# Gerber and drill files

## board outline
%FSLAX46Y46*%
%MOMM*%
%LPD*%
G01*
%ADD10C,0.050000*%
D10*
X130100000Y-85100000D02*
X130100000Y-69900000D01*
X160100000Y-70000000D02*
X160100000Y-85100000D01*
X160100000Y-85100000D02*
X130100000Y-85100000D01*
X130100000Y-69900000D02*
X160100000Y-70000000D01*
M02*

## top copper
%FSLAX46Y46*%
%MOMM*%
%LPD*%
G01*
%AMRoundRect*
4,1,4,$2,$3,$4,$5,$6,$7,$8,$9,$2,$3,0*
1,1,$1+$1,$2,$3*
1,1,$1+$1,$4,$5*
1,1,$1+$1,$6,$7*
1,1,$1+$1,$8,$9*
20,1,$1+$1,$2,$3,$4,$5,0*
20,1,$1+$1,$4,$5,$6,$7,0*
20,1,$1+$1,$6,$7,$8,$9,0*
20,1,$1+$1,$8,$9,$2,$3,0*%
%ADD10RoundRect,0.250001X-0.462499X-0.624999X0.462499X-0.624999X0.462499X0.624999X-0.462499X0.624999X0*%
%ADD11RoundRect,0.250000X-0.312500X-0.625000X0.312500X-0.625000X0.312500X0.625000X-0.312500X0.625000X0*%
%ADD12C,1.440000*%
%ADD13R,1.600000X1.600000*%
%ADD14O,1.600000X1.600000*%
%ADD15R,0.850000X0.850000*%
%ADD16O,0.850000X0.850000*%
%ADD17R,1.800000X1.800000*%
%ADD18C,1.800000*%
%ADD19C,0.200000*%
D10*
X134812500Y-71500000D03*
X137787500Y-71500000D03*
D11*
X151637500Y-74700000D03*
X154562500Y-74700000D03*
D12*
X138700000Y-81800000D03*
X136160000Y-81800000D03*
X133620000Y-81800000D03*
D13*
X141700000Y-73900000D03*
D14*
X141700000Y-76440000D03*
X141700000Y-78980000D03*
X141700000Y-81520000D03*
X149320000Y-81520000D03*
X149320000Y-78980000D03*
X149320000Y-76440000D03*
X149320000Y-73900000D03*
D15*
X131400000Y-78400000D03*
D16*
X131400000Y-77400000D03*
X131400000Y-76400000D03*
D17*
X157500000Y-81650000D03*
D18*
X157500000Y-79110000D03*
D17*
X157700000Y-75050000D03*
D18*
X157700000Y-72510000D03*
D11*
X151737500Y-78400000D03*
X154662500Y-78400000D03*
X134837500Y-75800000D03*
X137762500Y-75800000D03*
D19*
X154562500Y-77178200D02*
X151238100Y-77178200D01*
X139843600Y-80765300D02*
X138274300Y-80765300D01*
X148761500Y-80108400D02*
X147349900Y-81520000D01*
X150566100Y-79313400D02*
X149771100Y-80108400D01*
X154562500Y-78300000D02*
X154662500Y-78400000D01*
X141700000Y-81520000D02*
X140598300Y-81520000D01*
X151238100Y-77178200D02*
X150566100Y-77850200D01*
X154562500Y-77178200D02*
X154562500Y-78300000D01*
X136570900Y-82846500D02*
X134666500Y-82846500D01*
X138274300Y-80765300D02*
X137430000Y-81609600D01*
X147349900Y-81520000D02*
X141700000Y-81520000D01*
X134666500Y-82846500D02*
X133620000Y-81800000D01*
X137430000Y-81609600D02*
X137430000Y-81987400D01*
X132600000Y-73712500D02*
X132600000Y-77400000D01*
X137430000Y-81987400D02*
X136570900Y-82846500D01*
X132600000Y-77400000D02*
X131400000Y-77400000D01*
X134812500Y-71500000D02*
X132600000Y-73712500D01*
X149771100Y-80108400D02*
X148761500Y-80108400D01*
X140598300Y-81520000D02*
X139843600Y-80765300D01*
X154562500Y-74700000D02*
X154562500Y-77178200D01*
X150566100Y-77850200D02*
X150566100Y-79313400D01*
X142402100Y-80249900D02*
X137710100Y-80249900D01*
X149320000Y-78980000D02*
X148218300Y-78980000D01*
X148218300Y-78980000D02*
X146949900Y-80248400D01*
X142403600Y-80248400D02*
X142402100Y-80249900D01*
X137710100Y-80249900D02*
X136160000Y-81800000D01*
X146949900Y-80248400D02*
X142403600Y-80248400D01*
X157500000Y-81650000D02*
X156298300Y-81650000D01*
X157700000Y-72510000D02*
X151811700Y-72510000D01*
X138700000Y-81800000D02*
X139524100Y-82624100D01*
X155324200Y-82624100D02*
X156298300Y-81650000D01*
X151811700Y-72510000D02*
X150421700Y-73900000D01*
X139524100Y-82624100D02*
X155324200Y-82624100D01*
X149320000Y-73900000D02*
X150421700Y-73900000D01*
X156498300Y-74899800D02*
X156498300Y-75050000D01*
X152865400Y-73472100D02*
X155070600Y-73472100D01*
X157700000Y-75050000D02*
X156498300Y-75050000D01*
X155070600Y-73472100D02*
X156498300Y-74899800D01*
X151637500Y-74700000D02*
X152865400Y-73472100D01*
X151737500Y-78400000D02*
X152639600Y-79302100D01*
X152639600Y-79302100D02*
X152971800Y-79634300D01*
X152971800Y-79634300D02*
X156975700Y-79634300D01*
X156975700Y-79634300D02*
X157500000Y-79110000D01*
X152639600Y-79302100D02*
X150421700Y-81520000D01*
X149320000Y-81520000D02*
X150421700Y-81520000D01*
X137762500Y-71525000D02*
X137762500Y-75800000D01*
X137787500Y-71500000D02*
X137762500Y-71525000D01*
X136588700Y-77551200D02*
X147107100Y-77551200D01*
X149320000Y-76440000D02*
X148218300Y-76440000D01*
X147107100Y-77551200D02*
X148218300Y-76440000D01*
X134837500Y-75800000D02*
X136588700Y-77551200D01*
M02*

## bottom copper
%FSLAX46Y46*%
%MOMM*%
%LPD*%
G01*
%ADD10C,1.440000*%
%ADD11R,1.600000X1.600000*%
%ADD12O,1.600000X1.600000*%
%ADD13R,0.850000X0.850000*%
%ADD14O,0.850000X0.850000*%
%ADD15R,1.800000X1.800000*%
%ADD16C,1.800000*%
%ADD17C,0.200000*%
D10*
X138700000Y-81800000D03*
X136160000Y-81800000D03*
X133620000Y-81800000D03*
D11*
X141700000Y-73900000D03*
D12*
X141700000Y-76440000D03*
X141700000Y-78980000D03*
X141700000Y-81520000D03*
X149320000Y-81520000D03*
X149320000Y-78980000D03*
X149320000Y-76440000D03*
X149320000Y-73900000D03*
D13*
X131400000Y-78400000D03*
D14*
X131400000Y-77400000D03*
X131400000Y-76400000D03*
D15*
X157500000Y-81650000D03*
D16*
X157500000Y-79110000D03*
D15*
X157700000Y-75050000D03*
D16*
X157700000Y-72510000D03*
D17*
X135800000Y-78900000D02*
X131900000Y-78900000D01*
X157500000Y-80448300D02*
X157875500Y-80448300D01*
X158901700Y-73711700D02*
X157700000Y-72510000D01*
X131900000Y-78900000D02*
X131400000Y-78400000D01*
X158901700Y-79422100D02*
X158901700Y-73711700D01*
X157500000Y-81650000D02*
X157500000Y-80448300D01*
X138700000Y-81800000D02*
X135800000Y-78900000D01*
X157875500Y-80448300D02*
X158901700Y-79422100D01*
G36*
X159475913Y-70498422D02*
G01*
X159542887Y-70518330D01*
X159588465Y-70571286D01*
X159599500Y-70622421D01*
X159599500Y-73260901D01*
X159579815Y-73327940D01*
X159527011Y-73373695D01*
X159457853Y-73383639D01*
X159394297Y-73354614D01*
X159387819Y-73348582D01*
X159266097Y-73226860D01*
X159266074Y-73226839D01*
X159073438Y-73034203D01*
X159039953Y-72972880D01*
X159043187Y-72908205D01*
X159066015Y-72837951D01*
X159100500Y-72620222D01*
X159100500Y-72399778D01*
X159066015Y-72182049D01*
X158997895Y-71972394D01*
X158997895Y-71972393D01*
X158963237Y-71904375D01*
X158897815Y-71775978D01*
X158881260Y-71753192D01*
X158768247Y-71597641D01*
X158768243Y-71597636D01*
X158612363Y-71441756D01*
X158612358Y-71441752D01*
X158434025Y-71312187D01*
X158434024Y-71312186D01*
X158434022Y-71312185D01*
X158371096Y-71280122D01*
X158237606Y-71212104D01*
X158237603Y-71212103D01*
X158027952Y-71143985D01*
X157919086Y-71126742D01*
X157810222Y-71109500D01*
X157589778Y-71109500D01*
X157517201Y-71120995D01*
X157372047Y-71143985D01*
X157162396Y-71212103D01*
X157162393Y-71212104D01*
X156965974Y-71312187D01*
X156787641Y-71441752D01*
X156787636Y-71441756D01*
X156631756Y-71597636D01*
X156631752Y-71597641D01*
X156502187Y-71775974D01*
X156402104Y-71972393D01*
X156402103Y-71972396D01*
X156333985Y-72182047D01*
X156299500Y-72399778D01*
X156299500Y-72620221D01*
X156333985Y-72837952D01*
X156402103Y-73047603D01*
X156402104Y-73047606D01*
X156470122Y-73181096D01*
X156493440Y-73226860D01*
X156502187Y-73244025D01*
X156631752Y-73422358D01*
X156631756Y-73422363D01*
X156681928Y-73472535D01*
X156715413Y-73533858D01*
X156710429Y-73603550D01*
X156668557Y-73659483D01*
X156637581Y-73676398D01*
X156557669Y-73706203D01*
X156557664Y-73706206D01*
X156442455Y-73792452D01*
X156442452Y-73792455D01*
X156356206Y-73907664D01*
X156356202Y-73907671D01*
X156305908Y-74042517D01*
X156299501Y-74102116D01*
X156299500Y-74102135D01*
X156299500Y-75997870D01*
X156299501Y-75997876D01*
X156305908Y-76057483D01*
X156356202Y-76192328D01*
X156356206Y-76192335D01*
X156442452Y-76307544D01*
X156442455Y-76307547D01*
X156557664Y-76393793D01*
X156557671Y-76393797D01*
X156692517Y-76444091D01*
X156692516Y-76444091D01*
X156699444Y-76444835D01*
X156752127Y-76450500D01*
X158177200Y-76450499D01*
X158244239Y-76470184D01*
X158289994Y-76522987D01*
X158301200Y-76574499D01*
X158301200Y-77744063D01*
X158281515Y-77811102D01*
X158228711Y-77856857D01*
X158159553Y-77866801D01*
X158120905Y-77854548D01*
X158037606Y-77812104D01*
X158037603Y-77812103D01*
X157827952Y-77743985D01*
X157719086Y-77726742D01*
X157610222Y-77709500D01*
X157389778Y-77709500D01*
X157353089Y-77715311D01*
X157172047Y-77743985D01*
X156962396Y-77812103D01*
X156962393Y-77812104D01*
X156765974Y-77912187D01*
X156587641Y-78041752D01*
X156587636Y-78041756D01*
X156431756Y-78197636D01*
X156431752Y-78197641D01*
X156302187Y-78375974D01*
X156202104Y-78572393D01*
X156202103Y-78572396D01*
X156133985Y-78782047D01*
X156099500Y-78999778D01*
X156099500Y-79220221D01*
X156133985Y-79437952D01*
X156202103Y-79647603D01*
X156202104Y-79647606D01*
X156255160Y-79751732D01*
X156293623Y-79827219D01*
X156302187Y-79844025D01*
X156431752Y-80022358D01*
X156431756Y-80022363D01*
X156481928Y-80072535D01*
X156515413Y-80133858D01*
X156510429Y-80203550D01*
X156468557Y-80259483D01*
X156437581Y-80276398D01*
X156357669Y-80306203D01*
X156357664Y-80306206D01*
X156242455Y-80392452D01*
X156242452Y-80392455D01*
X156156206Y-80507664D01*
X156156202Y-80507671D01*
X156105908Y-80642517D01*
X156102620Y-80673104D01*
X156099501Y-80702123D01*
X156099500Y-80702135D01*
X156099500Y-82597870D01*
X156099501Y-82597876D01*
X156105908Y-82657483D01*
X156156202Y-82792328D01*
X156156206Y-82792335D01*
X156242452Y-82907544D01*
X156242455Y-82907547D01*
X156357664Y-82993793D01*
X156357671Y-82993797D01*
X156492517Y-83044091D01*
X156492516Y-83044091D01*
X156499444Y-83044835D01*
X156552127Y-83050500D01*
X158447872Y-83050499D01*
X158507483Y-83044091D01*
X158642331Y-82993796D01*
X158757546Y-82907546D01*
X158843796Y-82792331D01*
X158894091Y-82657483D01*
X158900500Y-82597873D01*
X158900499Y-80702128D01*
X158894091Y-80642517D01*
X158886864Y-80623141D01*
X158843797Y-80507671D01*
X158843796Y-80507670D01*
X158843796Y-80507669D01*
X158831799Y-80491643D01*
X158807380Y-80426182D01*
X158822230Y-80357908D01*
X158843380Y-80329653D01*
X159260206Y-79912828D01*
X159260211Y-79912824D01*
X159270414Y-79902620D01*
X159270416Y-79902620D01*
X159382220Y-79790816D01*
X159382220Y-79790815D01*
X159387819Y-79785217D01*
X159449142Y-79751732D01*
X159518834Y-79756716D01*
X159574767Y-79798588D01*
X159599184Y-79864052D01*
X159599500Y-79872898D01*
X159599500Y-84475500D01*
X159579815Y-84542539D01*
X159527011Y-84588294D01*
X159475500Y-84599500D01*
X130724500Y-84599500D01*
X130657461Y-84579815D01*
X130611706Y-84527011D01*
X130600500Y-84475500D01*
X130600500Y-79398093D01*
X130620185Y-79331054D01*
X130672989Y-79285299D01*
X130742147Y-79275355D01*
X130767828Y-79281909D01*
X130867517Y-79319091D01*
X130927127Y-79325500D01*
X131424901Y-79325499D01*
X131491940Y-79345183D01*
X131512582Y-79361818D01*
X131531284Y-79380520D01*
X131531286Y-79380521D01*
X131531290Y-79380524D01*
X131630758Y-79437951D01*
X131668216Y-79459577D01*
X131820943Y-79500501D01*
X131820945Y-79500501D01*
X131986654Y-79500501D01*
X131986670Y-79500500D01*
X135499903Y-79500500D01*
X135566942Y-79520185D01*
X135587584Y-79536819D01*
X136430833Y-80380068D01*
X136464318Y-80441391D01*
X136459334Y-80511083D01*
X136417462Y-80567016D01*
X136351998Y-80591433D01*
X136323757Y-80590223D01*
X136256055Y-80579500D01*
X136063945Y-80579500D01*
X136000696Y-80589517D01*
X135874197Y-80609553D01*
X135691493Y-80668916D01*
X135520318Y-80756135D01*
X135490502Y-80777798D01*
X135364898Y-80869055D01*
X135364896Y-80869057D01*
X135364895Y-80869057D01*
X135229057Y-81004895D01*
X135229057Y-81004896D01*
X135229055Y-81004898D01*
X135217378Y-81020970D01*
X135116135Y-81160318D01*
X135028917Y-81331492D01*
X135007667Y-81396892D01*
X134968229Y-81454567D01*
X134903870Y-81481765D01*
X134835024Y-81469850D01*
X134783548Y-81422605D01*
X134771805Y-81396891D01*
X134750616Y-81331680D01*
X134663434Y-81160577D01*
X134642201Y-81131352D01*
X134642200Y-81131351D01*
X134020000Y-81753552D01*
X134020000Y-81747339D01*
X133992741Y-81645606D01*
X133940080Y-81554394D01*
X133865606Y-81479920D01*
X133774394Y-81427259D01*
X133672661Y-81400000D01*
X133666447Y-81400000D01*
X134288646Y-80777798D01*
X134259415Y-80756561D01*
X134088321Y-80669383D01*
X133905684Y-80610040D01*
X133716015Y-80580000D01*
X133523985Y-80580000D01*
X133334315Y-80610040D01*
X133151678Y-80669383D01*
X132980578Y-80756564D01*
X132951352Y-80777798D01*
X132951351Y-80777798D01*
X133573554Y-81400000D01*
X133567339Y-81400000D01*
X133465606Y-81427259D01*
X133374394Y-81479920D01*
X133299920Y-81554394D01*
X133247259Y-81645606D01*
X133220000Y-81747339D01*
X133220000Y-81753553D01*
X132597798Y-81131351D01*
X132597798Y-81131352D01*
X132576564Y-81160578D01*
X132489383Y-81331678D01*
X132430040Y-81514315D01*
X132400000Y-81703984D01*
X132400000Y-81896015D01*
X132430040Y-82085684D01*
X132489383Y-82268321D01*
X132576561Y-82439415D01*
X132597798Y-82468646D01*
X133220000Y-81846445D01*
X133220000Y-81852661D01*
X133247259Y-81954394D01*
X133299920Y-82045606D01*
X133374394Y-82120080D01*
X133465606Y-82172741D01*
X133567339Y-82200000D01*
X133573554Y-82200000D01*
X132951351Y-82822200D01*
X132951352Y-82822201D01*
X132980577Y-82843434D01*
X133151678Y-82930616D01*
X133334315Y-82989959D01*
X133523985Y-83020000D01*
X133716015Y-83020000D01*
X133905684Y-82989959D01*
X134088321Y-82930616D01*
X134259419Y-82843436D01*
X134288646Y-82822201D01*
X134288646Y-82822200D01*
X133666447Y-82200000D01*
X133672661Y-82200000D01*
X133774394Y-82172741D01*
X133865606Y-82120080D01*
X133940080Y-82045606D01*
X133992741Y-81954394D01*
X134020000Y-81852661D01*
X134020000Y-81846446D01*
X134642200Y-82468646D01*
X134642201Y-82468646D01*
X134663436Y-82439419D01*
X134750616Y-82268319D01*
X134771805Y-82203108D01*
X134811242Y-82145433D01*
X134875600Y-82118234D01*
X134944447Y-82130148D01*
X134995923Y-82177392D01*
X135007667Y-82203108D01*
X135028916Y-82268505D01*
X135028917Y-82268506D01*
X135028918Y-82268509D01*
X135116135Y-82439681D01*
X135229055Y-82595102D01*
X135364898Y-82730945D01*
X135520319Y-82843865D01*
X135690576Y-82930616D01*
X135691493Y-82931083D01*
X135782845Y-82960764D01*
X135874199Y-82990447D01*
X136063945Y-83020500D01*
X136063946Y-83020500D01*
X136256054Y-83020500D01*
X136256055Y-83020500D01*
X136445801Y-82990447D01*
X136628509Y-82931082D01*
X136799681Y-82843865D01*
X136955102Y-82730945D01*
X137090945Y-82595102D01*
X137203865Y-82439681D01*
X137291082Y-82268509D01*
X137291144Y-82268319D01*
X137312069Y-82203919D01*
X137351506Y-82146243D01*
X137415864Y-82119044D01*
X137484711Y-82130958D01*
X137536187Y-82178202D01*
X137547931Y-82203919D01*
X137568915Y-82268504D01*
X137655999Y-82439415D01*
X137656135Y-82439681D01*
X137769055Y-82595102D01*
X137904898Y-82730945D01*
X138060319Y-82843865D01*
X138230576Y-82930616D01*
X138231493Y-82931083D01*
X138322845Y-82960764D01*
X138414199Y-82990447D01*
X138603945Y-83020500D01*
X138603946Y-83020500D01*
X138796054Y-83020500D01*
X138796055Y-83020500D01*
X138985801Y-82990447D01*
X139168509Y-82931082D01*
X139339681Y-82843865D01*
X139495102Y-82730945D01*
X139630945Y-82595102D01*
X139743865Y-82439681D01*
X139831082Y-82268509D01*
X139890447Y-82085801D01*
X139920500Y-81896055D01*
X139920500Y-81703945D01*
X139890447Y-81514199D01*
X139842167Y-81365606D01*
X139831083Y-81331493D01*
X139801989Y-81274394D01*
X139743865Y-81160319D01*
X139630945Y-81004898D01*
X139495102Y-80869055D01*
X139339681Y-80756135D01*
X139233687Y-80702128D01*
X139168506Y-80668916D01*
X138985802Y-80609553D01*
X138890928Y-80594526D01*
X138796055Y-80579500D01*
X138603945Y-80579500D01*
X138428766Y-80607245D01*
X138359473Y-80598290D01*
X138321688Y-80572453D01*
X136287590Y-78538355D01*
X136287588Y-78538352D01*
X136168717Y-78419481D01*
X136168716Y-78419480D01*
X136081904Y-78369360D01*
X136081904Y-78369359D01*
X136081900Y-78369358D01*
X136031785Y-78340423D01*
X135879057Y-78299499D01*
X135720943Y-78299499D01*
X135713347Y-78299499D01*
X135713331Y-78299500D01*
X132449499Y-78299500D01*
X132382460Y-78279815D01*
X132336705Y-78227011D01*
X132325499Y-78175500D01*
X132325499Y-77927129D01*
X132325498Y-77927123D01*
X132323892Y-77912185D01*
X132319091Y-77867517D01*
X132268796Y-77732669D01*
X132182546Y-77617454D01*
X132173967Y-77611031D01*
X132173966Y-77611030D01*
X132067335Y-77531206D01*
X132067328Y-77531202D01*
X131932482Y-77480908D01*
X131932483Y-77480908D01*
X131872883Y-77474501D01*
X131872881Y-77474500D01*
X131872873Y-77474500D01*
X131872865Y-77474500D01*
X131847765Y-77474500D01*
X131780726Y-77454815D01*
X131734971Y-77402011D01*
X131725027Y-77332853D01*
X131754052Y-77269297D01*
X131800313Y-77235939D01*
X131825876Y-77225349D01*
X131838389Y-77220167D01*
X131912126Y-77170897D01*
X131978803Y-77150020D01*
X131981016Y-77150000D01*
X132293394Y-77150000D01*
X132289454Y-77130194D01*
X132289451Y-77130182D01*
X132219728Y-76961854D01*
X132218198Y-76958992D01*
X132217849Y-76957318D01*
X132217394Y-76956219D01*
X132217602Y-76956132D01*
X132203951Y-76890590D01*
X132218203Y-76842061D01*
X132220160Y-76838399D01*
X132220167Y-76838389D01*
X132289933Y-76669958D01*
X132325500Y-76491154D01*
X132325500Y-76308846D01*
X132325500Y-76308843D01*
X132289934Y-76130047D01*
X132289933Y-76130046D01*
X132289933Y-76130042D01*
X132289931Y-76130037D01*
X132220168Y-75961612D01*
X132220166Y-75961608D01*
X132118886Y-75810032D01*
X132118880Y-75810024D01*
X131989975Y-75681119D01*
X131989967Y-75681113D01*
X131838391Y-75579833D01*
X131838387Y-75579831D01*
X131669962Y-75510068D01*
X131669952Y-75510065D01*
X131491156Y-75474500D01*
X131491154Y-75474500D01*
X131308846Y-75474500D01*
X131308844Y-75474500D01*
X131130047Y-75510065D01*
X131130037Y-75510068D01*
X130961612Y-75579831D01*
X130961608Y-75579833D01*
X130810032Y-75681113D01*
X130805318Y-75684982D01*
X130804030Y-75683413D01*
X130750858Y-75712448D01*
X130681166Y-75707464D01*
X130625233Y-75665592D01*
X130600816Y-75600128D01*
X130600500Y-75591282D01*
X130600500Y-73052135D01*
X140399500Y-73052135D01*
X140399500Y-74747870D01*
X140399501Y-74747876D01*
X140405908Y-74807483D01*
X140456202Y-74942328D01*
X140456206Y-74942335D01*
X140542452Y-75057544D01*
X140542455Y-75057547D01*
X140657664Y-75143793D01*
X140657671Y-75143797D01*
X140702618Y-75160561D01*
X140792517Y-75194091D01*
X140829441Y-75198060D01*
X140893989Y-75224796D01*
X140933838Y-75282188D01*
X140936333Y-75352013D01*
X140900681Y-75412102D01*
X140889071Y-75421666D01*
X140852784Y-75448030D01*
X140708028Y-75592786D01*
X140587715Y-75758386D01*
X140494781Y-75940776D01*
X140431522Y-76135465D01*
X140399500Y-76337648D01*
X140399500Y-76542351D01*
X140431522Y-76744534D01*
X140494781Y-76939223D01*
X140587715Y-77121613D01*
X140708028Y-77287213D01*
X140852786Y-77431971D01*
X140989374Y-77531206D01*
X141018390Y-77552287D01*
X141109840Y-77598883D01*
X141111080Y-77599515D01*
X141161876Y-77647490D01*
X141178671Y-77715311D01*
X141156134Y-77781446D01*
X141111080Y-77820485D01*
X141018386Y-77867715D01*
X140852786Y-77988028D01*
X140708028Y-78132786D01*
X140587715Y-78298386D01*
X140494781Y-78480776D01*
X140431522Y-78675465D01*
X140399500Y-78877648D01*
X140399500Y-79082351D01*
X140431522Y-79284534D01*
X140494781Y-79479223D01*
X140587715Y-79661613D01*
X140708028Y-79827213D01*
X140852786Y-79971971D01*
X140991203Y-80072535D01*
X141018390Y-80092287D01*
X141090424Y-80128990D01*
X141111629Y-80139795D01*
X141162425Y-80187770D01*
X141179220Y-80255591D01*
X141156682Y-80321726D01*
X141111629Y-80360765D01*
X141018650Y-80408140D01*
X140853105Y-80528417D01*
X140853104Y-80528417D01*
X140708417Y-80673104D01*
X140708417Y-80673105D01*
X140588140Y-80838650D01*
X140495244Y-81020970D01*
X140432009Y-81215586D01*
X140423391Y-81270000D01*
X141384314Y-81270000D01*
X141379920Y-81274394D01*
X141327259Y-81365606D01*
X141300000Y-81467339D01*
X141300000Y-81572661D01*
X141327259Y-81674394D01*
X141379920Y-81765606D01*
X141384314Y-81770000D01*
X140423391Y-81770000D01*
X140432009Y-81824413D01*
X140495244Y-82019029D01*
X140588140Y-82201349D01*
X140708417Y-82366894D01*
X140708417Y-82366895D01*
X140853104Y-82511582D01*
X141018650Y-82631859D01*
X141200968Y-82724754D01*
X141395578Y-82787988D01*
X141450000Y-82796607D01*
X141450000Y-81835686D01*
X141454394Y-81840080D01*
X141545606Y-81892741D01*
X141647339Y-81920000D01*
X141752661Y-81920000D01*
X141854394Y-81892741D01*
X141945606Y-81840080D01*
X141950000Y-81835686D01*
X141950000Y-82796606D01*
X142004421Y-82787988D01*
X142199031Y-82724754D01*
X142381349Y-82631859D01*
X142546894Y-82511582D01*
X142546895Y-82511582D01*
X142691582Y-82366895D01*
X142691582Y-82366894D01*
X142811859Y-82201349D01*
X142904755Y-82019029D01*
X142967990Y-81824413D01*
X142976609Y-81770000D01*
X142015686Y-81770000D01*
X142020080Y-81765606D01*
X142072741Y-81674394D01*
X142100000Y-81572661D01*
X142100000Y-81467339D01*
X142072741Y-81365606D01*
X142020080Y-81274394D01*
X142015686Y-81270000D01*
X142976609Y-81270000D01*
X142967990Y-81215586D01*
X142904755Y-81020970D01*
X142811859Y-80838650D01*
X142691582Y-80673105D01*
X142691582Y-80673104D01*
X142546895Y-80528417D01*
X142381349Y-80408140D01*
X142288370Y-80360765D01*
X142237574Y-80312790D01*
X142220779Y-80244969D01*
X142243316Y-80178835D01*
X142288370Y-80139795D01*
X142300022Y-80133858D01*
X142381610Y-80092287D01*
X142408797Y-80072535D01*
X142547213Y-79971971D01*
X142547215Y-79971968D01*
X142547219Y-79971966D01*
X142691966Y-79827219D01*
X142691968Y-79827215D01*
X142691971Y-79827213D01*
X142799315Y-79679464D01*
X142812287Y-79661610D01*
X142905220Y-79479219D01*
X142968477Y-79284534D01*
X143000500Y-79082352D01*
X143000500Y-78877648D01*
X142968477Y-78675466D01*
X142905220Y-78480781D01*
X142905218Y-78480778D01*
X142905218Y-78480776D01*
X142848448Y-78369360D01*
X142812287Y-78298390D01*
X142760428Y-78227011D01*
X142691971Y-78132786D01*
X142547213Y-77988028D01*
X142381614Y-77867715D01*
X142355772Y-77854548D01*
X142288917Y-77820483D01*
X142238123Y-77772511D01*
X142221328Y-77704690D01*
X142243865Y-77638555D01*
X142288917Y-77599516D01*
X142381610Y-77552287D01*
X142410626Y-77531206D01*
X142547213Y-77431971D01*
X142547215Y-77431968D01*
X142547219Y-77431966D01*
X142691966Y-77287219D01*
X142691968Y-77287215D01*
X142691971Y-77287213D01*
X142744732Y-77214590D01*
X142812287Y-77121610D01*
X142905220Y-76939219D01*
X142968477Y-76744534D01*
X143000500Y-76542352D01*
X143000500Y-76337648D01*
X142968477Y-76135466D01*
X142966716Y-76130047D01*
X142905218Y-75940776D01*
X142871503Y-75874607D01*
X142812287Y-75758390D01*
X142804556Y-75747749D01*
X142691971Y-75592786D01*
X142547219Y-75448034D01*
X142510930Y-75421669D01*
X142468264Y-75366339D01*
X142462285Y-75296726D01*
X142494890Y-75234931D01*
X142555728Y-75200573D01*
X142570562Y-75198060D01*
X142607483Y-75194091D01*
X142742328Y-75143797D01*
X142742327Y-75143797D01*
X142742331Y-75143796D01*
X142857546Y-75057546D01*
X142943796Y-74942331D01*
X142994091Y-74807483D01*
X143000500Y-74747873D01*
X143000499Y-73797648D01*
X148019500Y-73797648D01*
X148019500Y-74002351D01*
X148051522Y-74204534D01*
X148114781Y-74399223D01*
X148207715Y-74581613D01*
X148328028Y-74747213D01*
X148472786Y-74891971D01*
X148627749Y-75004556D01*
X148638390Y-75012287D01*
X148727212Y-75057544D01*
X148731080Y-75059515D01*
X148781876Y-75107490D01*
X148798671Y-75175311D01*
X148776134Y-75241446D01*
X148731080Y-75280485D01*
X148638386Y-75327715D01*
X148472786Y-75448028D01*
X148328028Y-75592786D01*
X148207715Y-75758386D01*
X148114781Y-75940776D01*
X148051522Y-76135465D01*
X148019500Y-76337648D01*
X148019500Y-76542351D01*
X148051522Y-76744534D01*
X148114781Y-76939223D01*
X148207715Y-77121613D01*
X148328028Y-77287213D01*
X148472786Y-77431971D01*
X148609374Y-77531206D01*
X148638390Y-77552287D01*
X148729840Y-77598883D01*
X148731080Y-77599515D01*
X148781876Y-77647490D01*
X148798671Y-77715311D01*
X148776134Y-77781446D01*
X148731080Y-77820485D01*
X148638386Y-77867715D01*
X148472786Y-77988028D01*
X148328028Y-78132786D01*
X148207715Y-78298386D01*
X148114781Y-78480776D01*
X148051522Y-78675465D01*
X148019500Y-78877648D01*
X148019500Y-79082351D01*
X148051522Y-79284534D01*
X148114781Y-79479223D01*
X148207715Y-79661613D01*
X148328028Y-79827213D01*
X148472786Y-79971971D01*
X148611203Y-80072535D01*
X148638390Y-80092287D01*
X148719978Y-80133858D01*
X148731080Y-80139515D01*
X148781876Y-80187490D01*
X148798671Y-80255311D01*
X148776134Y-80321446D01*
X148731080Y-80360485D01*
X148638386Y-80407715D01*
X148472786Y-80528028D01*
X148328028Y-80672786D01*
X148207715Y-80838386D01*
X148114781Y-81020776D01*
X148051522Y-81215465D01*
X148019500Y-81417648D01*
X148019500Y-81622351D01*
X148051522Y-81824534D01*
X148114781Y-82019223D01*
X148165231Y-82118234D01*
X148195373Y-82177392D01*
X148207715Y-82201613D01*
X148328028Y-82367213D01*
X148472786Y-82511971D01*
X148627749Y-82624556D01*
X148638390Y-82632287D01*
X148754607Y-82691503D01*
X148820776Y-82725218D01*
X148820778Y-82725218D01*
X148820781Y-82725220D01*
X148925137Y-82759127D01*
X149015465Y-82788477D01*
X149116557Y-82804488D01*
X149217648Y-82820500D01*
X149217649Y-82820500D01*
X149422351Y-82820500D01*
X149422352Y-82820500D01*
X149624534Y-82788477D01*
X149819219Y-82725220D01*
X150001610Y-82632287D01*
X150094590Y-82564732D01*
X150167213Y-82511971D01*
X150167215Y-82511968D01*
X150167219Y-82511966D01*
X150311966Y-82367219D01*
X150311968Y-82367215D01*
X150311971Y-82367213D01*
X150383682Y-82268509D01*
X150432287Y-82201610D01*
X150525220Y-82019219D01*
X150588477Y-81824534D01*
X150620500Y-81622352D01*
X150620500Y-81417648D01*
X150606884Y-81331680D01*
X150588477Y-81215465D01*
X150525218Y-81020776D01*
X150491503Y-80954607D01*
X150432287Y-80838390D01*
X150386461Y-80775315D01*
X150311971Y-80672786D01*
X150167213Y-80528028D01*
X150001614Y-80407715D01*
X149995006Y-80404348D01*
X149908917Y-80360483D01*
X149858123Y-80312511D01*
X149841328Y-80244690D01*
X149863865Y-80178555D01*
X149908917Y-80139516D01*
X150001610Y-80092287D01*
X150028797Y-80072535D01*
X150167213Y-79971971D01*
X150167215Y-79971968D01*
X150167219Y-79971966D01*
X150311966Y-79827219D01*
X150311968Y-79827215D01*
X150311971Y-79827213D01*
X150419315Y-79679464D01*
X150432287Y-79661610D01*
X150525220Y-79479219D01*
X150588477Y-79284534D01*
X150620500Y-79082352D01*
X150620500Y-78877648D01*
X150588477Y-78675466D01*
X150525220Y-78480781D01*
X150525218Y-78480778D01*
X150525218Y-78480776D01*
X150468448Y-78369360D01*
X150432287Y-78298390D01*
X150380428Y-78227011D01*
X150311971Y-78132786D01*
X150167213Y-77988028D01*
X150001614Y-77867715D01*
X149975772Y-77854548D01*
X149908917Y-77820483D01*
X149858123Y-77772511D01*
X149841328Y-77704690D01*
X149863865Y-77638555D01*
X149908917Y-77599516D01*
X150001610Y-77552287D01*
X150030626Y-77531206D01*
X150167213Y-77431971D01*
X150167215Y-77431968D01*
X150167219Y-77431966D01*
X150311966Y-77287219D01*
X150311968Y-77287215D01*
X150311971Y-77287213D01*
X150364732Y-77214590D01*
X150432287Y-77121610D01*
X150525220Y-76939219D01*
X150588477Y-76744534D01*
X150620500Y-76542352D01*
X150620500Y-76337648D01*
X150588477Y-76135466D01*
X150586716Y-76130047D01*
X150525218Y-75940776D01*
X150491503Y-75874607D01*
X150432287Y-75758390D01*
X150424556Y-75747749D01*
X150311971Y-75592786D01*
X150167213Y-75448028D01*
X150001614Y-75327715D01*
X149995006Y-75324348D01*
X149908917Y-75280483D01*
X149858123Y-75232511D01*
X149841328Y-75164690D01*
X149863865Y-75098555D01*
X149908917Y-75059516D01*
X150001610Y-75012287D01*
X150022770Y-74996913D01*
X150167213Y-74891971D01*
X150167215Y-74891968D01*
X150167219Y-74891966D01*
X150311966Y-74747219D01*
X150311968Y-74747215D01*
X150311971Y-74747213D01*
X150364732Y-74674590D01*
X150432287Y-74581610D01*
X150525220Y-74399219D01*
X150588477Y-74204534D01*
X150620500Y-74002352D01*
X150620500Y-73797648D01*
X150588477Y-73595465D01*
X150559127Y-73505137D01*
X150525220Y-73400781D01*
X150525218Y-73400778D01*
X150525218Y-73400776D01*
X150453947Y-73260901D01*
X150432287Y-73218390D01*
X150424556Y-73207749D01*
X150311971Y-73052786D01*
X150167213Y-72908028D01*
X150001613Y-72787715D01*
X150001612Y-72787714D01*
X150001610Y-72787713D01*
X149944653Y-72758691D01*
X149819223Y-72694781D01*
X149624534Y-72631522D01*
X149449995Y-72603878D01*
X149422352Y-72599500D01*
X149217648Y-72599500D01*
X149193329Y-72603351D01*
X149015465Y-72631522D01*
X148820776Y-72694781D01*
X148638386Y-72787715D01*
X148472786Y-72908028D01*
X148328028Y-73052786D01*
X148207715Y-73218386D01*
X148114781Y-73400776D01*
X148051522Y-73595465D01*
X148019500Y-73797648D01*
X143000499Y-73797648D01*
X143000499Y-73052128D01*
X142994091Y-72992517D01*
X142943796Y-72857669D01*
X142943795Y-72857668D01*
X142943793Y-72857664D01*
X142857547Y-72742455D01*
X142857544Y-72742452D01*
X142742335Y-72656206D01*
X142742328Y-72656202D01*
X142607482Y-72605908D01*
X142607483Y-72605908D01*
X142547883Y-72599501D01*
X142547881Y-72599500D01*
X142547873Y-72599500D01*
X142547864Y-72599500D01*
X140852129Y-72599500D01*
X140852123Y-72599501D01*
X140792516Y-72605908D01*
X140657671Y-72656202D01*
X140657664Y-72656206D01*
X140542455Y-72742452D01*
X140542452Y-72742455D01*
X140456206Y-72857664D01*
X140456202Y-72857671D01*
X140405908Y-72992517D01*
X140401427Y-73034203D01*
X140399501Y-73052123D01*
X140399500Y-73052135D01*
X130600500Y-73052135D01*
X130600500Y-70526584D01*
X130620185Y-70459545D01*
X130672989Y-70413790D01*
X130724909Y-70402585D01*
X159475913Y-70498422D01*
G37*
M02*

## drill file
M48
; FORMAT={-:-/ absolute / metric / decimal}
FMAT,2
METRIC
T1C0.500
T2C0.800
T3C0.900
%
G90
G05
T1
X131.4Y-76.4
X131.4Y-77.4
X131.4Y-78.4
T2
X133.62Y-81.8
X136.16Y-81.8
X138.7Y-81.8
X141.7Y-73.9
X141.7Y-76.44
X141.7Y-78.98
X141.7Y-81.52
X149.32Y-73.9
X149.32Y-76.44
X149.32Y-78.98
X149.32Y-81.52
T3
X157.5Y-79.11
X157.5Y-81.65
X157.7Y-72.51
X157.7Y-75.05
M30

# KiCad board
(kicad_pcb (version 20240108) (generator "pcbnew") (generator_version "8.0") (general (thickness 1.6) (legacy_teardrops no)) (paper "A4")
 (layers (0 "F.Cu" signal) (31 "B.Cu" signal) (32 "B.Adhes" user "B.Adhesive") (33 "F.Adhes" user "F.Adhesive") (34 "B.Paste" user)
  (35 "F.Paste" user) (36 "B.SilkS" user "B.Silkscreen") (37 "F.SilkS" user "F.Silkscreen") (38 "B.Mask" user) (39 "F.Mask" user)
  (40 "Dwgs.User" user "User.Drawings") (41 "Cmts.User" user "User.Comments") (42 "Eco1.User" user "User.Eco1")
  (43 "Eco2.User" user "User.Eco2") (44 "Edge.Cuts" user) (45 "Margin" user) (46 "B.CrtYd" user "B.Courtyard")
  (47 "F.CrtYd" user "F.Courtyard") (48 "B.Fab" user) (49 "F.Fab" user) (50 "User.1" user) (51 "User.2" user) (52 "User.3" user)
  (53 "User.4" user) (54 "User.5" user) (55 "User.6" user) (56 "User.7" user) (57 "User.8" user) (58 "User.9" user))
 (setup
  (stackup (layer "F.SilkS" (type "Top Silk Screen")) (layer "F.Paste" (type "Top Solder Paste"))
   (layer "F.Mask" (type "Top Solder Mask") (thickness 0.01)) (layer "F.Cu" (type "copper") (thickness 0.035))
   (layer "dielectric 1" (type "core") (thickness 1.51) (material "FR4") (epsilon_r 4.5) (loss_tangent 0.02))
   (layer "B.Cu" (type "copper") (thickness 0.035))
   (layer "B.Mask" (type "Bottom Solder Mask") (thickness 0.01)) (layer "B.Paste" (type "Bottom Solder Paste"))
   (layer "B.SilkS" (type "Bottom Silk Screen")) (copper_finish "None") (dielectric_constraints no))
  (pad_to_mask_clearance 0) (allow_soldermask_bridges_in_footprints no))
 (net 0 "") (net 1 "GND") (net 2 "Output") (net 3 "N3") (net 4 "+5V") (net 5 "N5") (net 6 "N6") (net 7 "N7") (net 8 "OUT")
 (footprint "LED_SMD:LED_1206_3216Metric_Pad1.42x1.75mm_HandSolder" (layer "F.Cu") (at 136.3 71.5)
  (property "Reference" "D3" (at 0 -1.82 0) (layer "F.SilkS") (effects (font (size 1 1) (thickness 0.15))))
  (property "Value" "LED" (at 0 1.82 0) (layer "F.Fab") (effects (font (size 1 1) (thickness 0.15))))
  (pad "1" smd roundrect (at -1.4875 0) (size 1.425 1.75) (layers "F.Cu" "F.Paste" "F.Mask") (roundrect_rratio 0.175439) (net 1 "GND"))
  (pad "2" smd roundrect (at 1.4875 0) (size 1.425 1.75) (layers "F.Cu" "F.Paste" "F.Mask") (roundrect_rratio 0.175439) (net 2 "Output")))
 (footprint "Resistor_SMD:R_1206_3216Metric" (layer "F.Cu") (at 153.1 74.7)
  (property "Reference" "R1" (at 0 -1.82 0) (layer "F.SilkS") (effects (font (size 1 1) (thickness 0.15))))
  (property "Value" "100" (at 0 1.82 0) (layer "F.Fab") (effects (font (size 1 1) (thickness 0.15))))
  (pad "1" smd roundrect (at -1.4625 0) (size 1.125 1.75) (layers "F.Cu" "F.Paste" "F.Mask") (roundrect_rratio 0.222222) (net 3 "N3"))
  (pad "2" smd roundrect (at 1.4625 0) (size 1.125 1.75) (layers "F.Cu" "F.Paste" "F.Mask") (roundrect_rratio 0.222222) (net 1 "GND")))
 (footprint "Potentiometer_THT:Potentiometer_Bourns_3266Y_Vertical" (layer "F.Cu") (at 138.7 81.8)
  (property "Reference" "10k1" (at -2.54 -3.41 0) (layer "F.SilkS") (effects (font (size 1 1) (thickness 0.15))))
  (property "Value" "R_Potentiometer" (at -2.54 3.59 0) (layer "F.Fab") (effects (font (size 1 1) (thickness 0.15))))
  (pad "1" thru_hole circle (at 0 0) (size 1.44 1.44) (drill 0.8) (layers "*.Cu" "*.Mask") (remove_unused_layers no) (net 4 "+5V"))
  (pad "2" thru_hole circle (at -2.54 0) (size 1.44 1.44) (drill 0.8) (layers "*.Cu" "*.Mask") (remove_unused_layers no) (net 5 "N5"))
  (pad "3" thru_hole circle (at -5.08 0) (size 1.44 1.44) (drill 0.8) (layers "*.Cu" "*.Mask") (remove_unused_layers no) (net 1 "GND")))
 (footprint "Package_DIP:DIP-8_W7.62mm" (layer "F.Cu") (at 141.7 73.9)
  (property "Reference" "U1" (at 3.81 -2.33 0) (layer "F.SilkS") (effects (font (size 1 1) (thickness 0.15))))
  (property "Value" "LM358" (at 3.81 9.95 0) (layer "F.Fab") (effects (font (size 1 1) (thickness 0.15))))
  (pad "1" thru_hole rect (at 0 0) (size 1.6 1.6) (drill 0.8) (layers "*.Cu" "*.Mask") (remove_unused_layers no))
  (pad "2" thru_hole oval (at 0 2.54) (size 1.6 1.6) (drill 0.8) (layers "*.Cu" "*.Mask") (remove_unused_layers no))
  (pad "3" thru_hole oval (at 0 5.08) (size 1.6 1.6) (drill 0.8) (layers "*.Cu" "*.Mask") (remove_unused_layers no))
  (pad "4" thru_hole oval (at 0 7.62) (size 1.6 1.6) (drill 0.8) (layers "*.Cu" "*.Mask") (remove_unused_layers no) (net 1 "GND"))
  (pad "5" thru_hole oval (at 7.62 7.62) (size 1.6 1.6) (drill 0.8) (layers "*.Cu" "*.Mask") (remove_unused_layers no) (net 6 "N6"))
  (pad "6" thru_hole oval (at 7.62 5.08) (size 1.6 1.6) (drill 0.8) (layers "*.Cu" "*.Mask") (remove_unused_layers no) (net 5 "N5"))
  (pad "7" thru_hole oval (at 7.62 2.54) (size 1.6 1.6) (drill 0.8) (layers "*.Cu" "*.Mask") (remove_unused_layers no) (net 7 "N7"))
  (pad "8" thru_hole oval (at 7.62 0) (size 1.6 1.6) (drill 0.8) (layers "*.Cu" "*.Mask") (remove_unused_layers no) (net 4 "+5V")))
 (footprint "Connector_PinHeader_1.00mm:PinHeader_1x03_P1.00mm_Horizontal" (layer "F.Cu") (at 131.4 78.4 180)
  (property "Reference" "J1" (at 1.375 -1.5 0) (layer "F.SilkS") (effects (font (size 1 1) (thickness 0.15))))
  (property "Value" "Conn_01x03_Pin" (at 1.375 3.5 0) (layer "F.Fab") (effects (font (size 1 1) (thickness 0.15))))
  (pad "1" thru_hole rect (at 0 0 180) (size 0.85 0.85) (drill 0.5) (layers "*.Cu" "*.Mask") (remove_unused_layers no) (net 4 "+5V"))
  (pad "2" thru_hole oval (at 0 1 180) (size 0.85 0.85) (drill 0.5) (layers "*.Cu" "*.Mask") (remove_unused_layers no) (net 1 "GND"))
  (pad "3" thru_hole oval (at 0 2 180) (size 0.85 0.85) (drill 0.5) (layers "*.Cu" "*.Mask") (remove_unused_layers no) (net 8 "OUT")))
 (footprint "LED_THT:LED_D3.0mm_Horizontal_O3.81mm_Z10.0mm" (layer "F.Cu") (at 157.5 81.65 90)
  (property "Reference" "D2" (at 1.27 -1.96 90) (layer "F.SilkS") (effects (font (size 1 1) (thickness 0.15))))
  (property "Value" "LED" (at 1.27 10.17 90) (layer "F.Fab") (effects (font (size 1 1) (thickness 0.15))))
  (pad "1" thru_hole rect (at 0 0 90) (size 1.8 1.8) (drill 0.9) (layers "*.Cu" "*.Mask") (remove_unused_layers no) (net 4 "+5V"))
  (pad "2" thru_hole circle (at 2.54 0 90) (size 1.8 1.8) (drill 0.9) (layers "*.Cu" "*.Mask") (remove_unused_layers no) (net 6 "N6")))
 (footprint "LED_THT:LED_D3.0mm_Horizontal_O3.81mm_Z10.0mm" (layer "F.Cu") (at 157.7 75.05 90)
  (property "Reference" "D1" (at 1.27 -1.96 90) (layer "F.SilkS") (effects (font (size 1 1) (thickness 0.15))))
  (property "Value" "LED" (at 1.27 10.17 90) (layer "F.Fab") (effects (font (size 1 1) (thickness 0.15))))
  (pad "1" thru_hole rect (at 0 0 90) (size 1.8 1.8) (drill 0.9) (layers "*.Cu" "*.Mask") (remove_unused_layers no) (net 3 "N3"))
  (pad "2" thru_hole circle (at 2.54 0 90) (size 1.8 1.8) (drill 0.9) (layers "*.Cu" "*.Mask") (remove_unused_layers no) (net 4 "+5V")))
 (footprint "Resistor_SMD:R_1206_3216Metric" (layer "F.Cu") (at 153.2 78.4)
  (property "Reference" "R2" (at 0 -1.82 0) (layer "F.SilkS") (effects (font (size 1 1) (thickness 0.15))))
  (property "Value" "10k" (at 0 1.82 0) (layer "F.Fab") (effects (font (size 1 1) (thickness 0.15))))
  (pad "1" smd roundrect (at -1.4625 0) (size 1.125 1.75) (layers "F.Cu" "F.Paste" "F.Mask") (roundrect_rratio 0.222222) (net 6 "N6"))
  (pad "2" smd roundrect (at 1.4625 0) (size 1.125 1.75) (layers "F.Cu" "F.Paste" "F.Mask") (roundrect_rratio 0.222222) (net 1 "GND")))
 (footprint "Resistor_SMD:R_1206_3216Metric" (layer "F.Cu") (at 136.3 75.8)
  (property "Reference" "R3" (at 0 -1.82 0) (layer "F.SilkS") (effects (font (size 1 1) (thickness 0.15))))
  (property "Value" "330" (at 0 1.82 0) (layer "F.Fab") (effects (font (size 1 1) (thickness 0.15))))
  (pad "1" smd roundrect (at -1.4625 0) (size 1.125 1.75) (layers "F.Cu" "F.Paste" "F.Mask") (roundrect_rratio 0.222222) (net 7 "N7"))
  (pad "2" smd roundrect (at 1.4625 0) (size 1.125 1.75) (layers "F.Cu" "F.Paste" "F.Mask") (roundrect_rratio 0.222222) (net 2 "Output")))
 (gr_line (start 130.1 85.1) (end 130.1 69.9) (stroke (width 0.05) (type default)) (layer "Edge.Cuts"))
 (gr_line (start 160.1 70) (end 160.1 85.1) (stroke (width 0.05) (type default)) (layer "Edge.Cuts"))
 (gr_line (start 160.1 85.1) (end 130.1 85.1) (stroke (width 0.05) (type default)) (layer "Edge.Cuts"))
 (gr_line (start 130.1 69.9) (end 160.1 70) (stroke (width 0.05) (type default)) (layer "Edge.Cuts"))
 (segment (start 154.5625 77.1782) (end 151.2381 77.1782) (width 0.2) (layer "F.Cu") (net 1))
 (segment (start 139.8436 80.7653) (end 138.2743 80.7653) (width 0.2) (layer "F.Cu") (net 1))
 (segment (start 148.7615 80.1084) (end 147.3499 81.52) (width 0.2) (layer "F.Cu") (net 1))
 (segment (start 150.5661 79.3134) (end 149.7711 80.1084) (width 0.2) (layer "F.Cu") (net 1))
 (segment (start 154.5625 78.3) (end 154.6625 78.4) (width 0.2) (layer "F.Cu") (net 1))
 (segment (start 141.7 81.52) (end 140.5983 81.52) (width 0.2) (layer "F.Cu") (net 1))
 (segment (start 151.2381 77.1782) (end 150.5661 77.8502) (width 0.2) (layer "F.Cu") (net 1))
 (segment (start 154.5625 77.1782) (end 154.5625 78.3) (width 0.2) (layer "F.Cu") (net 1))
 (segment (start 136.5709 82.8465) (end 134.6665 82.8465) (width 0.2) (layer "F.Cu") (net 1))
 (segment (start 138.2743 80.7653) (end 137.43 81.6096) (width 0.2) (layer "F.Cu") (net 1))
 (segment (start 147.3499 81.52) (end 141.7 81.52) (width 0.2) (layer "F.Cu") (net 1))
 (segment (start 134.6665 82.8465) (end 133.62 81.8) (width 0.2) (layer "F.Cu") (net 1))
 (segment (start 137.43 81.6096) (end 137.43 81.9874) (width 0.2) (layer "F.Cu") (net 1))
 (segment (start 132.6 73.7125) (end 132.6 77.4) (width 0.2) (layer "F.Cu") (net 1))
 (segment (start 137.43 81.9874) (end 136.5709 82.8465) (width 0.2) (layer "F.Cu") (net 1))
 (segment (start 132.6 77.4) (end 131.4 77.4) (width 0.2) (layer "F.Cu") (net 1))
 (segment (start 134.8125 71.5) (end 132.6 73.7125) (width 0.2) (layer "F.Cu") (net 1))
 (segment (start 149.7711 80.1084) (end 148.7615 80.1084) (width 0.2) (layer "F.Cu") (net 1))
 (segment (start 140.5983 81.52) (end 139.8436 80.7653) (width 0.2) (layer "F.Cu") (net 1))
 (segment (start 154.5625 74.7) (end 154.5625 77.1782) (width 0.2) (layer "F.Cu") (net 1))
 (segment (start 150.5661 77.8502) (end 150.5661 79.3134) (width 0.2) (layer "F.Cu") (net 1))
 (segment (start 142.4021 80.2499) (end 137.7101 80.2499) (width 0.2) (layer "F.Cu") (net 5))
 (segment (start 149.32 78.98) (end 148.2183 78.98) (width 0.2) (layer "F.Cu") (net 5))
 (segment (start 148.2183 78.98) (end 146.9499 80.2484) (width 0.2) (layer "F.Cu") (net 5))
 (segment (start 142.4036 80.2484) (end 142.4021 80.2499) (width 0.2) (layer "F.Cu") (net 5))
 (segment (start 137.7101 80.2499) (end 136.16 81.8) (width 0.2) (layer "F.Cu") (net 5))
 (segment (start 146.9499 80.2484) (end 142.4036 80.2484) (width 0.2) (layer "F.Cu") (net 5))
 (segment (start 157.5 81.65) (end 156.2983 81.65) (width 0.2) (layer "F.Cu") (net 4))
 (segment (start 157.7 72.51) (end 151.8117 72.51) (width 0.2) (layer "F.Cu") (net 4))
 (segment (start 138.7 81.8) (end 139.5241 82.6241) (width 0.2) (layer "F.Cu") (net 4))
 (segment (start 155.3242 82.6241) (end 156.2983 81.65) (width 0.2) (layer "F.Cu") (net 4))
 (segment (start 151.8117 72.51) (end 150.4217 73.9) (width 0.2) (layer "F.Cu") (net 4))
 (segment (start 139.5241 82.6241) (end 155.3242 82.6241) (width 0.2) (layer "F.Cu") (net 4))
 (segment (start 149.32 73.9) (end 150.4217 73.9) (width 0.2) (layer "F.Cu") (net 4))
 (segment (start 135.8 78.9) (end 131.9 78.9) (width 0.2) (layer "B.Cu") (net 4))
 (segment (start 157.5 80.4483) (end 157.8755 80.4483) (width 0.2) (layer "B.Cu") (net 4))
 (segment (start 158.9017 73.7117) (end 157.7 72.51) (width 0.2) (layer "B.Cu") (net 4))
 (segment (start 131.9 78.9) (end 131.4 78.4) (width 0.2) (layer "B.Cu") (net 4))
 (segment (start 158.9017 79.4221) (end 158.9017 73.7117) (width 0.2) (layer "B.Cu") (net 4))
 (segment (start 157.5 81.65) (end 157.5 80.4483) (width 0.2) (layer "B.Cu") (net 4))
 (segment (start 138.7 81.8) (end 135.8 78.9) (width 0.2) (layer "B.Cu") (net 4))
 (segment (start 157.8755 80.4483) (end 158.9017 79.4221) (width 0.2) (layer "B.Cu") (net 4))
 (segment (start 156.4983 74.8998) (end 156.4983 75.05) (width 0.2) (layer "F.Cu") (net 3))
 (segment (start 152.8654 73.4721) (end 155.0706 73.4721) (width 0.2) (layer "F.Cu") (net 3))
 (segment (start 157.7 75.05) (end 156.4983 75.05) (width 0.2) (layer "F.Cu") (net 3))
 (segment (start 155.0706 73.4721) (end 156.4983 74.8998) (width 0.2) (layer "F.Cu") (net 3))
 (segment (start 151.6375 74.7) (end 152.8654 73.4721) (width 0.2) (layer "F.Cu") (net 3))
 (segment (start 151.7375 78.4) (end 152.6396 79.3021) (width 0.2) (layer "F.Cu") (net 6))
 (segment (start 152.6396 79.3021) (end 152.9718 79.6343) (width 0.2) (layer "F.Cu") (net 6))
 (segment (start 152.9718 79.6343) (end 156.9757 79.6343) (width 0.2) (layer "F.Cu") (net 6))
 (segment (start 156.9757 79.6343) (end 157.5 79.11) (width 0.2) (layer "F.Cu") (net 6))
 (segment (start 152.6396 79.3021) (end 150.4217 81.52) (width 0.2) (layer "F.Cu") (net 6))
 (segment (start 149.32 81.52) (end 150.4217 81.52) (width 0.2) (layer "F.Cu") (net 6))
 (segment (start 137.7625 71.525) (end 137.7625 75.8) (width 0.2) (layer "F.Cu") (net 2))
 (segment (start 137.7875 71.5) (end 137.7625 71.525) (width 0.2) (layer "F.Cu") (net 2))
 (segment (start 136.5887 77.5512) (end 147.1071 77.5512) (width 0.2) (layer "F.Cu") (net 7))
 (segment (start 149.32 76.44) (end 148.2183 76.44) (width 0.2) (layer "F.Cu") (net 7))
 (segment (start 147.1071 77.5512) (end 148.2183 76.44) (width 0.2) (layer "F.Cu") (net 7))
 (segment (start 134.8375 75.8) (end 136.5887 77.5512) (width 0.2) (layer "F.Cu") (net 7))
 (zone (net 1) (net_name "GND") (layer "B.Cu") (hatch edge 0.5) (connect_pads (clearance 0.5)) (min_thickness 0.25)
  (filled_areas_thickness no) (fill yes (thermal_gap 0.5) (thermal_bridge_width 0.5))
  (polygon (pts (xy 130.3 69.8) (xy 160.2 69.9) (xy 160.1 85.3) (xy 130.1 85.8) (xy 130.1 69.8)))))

